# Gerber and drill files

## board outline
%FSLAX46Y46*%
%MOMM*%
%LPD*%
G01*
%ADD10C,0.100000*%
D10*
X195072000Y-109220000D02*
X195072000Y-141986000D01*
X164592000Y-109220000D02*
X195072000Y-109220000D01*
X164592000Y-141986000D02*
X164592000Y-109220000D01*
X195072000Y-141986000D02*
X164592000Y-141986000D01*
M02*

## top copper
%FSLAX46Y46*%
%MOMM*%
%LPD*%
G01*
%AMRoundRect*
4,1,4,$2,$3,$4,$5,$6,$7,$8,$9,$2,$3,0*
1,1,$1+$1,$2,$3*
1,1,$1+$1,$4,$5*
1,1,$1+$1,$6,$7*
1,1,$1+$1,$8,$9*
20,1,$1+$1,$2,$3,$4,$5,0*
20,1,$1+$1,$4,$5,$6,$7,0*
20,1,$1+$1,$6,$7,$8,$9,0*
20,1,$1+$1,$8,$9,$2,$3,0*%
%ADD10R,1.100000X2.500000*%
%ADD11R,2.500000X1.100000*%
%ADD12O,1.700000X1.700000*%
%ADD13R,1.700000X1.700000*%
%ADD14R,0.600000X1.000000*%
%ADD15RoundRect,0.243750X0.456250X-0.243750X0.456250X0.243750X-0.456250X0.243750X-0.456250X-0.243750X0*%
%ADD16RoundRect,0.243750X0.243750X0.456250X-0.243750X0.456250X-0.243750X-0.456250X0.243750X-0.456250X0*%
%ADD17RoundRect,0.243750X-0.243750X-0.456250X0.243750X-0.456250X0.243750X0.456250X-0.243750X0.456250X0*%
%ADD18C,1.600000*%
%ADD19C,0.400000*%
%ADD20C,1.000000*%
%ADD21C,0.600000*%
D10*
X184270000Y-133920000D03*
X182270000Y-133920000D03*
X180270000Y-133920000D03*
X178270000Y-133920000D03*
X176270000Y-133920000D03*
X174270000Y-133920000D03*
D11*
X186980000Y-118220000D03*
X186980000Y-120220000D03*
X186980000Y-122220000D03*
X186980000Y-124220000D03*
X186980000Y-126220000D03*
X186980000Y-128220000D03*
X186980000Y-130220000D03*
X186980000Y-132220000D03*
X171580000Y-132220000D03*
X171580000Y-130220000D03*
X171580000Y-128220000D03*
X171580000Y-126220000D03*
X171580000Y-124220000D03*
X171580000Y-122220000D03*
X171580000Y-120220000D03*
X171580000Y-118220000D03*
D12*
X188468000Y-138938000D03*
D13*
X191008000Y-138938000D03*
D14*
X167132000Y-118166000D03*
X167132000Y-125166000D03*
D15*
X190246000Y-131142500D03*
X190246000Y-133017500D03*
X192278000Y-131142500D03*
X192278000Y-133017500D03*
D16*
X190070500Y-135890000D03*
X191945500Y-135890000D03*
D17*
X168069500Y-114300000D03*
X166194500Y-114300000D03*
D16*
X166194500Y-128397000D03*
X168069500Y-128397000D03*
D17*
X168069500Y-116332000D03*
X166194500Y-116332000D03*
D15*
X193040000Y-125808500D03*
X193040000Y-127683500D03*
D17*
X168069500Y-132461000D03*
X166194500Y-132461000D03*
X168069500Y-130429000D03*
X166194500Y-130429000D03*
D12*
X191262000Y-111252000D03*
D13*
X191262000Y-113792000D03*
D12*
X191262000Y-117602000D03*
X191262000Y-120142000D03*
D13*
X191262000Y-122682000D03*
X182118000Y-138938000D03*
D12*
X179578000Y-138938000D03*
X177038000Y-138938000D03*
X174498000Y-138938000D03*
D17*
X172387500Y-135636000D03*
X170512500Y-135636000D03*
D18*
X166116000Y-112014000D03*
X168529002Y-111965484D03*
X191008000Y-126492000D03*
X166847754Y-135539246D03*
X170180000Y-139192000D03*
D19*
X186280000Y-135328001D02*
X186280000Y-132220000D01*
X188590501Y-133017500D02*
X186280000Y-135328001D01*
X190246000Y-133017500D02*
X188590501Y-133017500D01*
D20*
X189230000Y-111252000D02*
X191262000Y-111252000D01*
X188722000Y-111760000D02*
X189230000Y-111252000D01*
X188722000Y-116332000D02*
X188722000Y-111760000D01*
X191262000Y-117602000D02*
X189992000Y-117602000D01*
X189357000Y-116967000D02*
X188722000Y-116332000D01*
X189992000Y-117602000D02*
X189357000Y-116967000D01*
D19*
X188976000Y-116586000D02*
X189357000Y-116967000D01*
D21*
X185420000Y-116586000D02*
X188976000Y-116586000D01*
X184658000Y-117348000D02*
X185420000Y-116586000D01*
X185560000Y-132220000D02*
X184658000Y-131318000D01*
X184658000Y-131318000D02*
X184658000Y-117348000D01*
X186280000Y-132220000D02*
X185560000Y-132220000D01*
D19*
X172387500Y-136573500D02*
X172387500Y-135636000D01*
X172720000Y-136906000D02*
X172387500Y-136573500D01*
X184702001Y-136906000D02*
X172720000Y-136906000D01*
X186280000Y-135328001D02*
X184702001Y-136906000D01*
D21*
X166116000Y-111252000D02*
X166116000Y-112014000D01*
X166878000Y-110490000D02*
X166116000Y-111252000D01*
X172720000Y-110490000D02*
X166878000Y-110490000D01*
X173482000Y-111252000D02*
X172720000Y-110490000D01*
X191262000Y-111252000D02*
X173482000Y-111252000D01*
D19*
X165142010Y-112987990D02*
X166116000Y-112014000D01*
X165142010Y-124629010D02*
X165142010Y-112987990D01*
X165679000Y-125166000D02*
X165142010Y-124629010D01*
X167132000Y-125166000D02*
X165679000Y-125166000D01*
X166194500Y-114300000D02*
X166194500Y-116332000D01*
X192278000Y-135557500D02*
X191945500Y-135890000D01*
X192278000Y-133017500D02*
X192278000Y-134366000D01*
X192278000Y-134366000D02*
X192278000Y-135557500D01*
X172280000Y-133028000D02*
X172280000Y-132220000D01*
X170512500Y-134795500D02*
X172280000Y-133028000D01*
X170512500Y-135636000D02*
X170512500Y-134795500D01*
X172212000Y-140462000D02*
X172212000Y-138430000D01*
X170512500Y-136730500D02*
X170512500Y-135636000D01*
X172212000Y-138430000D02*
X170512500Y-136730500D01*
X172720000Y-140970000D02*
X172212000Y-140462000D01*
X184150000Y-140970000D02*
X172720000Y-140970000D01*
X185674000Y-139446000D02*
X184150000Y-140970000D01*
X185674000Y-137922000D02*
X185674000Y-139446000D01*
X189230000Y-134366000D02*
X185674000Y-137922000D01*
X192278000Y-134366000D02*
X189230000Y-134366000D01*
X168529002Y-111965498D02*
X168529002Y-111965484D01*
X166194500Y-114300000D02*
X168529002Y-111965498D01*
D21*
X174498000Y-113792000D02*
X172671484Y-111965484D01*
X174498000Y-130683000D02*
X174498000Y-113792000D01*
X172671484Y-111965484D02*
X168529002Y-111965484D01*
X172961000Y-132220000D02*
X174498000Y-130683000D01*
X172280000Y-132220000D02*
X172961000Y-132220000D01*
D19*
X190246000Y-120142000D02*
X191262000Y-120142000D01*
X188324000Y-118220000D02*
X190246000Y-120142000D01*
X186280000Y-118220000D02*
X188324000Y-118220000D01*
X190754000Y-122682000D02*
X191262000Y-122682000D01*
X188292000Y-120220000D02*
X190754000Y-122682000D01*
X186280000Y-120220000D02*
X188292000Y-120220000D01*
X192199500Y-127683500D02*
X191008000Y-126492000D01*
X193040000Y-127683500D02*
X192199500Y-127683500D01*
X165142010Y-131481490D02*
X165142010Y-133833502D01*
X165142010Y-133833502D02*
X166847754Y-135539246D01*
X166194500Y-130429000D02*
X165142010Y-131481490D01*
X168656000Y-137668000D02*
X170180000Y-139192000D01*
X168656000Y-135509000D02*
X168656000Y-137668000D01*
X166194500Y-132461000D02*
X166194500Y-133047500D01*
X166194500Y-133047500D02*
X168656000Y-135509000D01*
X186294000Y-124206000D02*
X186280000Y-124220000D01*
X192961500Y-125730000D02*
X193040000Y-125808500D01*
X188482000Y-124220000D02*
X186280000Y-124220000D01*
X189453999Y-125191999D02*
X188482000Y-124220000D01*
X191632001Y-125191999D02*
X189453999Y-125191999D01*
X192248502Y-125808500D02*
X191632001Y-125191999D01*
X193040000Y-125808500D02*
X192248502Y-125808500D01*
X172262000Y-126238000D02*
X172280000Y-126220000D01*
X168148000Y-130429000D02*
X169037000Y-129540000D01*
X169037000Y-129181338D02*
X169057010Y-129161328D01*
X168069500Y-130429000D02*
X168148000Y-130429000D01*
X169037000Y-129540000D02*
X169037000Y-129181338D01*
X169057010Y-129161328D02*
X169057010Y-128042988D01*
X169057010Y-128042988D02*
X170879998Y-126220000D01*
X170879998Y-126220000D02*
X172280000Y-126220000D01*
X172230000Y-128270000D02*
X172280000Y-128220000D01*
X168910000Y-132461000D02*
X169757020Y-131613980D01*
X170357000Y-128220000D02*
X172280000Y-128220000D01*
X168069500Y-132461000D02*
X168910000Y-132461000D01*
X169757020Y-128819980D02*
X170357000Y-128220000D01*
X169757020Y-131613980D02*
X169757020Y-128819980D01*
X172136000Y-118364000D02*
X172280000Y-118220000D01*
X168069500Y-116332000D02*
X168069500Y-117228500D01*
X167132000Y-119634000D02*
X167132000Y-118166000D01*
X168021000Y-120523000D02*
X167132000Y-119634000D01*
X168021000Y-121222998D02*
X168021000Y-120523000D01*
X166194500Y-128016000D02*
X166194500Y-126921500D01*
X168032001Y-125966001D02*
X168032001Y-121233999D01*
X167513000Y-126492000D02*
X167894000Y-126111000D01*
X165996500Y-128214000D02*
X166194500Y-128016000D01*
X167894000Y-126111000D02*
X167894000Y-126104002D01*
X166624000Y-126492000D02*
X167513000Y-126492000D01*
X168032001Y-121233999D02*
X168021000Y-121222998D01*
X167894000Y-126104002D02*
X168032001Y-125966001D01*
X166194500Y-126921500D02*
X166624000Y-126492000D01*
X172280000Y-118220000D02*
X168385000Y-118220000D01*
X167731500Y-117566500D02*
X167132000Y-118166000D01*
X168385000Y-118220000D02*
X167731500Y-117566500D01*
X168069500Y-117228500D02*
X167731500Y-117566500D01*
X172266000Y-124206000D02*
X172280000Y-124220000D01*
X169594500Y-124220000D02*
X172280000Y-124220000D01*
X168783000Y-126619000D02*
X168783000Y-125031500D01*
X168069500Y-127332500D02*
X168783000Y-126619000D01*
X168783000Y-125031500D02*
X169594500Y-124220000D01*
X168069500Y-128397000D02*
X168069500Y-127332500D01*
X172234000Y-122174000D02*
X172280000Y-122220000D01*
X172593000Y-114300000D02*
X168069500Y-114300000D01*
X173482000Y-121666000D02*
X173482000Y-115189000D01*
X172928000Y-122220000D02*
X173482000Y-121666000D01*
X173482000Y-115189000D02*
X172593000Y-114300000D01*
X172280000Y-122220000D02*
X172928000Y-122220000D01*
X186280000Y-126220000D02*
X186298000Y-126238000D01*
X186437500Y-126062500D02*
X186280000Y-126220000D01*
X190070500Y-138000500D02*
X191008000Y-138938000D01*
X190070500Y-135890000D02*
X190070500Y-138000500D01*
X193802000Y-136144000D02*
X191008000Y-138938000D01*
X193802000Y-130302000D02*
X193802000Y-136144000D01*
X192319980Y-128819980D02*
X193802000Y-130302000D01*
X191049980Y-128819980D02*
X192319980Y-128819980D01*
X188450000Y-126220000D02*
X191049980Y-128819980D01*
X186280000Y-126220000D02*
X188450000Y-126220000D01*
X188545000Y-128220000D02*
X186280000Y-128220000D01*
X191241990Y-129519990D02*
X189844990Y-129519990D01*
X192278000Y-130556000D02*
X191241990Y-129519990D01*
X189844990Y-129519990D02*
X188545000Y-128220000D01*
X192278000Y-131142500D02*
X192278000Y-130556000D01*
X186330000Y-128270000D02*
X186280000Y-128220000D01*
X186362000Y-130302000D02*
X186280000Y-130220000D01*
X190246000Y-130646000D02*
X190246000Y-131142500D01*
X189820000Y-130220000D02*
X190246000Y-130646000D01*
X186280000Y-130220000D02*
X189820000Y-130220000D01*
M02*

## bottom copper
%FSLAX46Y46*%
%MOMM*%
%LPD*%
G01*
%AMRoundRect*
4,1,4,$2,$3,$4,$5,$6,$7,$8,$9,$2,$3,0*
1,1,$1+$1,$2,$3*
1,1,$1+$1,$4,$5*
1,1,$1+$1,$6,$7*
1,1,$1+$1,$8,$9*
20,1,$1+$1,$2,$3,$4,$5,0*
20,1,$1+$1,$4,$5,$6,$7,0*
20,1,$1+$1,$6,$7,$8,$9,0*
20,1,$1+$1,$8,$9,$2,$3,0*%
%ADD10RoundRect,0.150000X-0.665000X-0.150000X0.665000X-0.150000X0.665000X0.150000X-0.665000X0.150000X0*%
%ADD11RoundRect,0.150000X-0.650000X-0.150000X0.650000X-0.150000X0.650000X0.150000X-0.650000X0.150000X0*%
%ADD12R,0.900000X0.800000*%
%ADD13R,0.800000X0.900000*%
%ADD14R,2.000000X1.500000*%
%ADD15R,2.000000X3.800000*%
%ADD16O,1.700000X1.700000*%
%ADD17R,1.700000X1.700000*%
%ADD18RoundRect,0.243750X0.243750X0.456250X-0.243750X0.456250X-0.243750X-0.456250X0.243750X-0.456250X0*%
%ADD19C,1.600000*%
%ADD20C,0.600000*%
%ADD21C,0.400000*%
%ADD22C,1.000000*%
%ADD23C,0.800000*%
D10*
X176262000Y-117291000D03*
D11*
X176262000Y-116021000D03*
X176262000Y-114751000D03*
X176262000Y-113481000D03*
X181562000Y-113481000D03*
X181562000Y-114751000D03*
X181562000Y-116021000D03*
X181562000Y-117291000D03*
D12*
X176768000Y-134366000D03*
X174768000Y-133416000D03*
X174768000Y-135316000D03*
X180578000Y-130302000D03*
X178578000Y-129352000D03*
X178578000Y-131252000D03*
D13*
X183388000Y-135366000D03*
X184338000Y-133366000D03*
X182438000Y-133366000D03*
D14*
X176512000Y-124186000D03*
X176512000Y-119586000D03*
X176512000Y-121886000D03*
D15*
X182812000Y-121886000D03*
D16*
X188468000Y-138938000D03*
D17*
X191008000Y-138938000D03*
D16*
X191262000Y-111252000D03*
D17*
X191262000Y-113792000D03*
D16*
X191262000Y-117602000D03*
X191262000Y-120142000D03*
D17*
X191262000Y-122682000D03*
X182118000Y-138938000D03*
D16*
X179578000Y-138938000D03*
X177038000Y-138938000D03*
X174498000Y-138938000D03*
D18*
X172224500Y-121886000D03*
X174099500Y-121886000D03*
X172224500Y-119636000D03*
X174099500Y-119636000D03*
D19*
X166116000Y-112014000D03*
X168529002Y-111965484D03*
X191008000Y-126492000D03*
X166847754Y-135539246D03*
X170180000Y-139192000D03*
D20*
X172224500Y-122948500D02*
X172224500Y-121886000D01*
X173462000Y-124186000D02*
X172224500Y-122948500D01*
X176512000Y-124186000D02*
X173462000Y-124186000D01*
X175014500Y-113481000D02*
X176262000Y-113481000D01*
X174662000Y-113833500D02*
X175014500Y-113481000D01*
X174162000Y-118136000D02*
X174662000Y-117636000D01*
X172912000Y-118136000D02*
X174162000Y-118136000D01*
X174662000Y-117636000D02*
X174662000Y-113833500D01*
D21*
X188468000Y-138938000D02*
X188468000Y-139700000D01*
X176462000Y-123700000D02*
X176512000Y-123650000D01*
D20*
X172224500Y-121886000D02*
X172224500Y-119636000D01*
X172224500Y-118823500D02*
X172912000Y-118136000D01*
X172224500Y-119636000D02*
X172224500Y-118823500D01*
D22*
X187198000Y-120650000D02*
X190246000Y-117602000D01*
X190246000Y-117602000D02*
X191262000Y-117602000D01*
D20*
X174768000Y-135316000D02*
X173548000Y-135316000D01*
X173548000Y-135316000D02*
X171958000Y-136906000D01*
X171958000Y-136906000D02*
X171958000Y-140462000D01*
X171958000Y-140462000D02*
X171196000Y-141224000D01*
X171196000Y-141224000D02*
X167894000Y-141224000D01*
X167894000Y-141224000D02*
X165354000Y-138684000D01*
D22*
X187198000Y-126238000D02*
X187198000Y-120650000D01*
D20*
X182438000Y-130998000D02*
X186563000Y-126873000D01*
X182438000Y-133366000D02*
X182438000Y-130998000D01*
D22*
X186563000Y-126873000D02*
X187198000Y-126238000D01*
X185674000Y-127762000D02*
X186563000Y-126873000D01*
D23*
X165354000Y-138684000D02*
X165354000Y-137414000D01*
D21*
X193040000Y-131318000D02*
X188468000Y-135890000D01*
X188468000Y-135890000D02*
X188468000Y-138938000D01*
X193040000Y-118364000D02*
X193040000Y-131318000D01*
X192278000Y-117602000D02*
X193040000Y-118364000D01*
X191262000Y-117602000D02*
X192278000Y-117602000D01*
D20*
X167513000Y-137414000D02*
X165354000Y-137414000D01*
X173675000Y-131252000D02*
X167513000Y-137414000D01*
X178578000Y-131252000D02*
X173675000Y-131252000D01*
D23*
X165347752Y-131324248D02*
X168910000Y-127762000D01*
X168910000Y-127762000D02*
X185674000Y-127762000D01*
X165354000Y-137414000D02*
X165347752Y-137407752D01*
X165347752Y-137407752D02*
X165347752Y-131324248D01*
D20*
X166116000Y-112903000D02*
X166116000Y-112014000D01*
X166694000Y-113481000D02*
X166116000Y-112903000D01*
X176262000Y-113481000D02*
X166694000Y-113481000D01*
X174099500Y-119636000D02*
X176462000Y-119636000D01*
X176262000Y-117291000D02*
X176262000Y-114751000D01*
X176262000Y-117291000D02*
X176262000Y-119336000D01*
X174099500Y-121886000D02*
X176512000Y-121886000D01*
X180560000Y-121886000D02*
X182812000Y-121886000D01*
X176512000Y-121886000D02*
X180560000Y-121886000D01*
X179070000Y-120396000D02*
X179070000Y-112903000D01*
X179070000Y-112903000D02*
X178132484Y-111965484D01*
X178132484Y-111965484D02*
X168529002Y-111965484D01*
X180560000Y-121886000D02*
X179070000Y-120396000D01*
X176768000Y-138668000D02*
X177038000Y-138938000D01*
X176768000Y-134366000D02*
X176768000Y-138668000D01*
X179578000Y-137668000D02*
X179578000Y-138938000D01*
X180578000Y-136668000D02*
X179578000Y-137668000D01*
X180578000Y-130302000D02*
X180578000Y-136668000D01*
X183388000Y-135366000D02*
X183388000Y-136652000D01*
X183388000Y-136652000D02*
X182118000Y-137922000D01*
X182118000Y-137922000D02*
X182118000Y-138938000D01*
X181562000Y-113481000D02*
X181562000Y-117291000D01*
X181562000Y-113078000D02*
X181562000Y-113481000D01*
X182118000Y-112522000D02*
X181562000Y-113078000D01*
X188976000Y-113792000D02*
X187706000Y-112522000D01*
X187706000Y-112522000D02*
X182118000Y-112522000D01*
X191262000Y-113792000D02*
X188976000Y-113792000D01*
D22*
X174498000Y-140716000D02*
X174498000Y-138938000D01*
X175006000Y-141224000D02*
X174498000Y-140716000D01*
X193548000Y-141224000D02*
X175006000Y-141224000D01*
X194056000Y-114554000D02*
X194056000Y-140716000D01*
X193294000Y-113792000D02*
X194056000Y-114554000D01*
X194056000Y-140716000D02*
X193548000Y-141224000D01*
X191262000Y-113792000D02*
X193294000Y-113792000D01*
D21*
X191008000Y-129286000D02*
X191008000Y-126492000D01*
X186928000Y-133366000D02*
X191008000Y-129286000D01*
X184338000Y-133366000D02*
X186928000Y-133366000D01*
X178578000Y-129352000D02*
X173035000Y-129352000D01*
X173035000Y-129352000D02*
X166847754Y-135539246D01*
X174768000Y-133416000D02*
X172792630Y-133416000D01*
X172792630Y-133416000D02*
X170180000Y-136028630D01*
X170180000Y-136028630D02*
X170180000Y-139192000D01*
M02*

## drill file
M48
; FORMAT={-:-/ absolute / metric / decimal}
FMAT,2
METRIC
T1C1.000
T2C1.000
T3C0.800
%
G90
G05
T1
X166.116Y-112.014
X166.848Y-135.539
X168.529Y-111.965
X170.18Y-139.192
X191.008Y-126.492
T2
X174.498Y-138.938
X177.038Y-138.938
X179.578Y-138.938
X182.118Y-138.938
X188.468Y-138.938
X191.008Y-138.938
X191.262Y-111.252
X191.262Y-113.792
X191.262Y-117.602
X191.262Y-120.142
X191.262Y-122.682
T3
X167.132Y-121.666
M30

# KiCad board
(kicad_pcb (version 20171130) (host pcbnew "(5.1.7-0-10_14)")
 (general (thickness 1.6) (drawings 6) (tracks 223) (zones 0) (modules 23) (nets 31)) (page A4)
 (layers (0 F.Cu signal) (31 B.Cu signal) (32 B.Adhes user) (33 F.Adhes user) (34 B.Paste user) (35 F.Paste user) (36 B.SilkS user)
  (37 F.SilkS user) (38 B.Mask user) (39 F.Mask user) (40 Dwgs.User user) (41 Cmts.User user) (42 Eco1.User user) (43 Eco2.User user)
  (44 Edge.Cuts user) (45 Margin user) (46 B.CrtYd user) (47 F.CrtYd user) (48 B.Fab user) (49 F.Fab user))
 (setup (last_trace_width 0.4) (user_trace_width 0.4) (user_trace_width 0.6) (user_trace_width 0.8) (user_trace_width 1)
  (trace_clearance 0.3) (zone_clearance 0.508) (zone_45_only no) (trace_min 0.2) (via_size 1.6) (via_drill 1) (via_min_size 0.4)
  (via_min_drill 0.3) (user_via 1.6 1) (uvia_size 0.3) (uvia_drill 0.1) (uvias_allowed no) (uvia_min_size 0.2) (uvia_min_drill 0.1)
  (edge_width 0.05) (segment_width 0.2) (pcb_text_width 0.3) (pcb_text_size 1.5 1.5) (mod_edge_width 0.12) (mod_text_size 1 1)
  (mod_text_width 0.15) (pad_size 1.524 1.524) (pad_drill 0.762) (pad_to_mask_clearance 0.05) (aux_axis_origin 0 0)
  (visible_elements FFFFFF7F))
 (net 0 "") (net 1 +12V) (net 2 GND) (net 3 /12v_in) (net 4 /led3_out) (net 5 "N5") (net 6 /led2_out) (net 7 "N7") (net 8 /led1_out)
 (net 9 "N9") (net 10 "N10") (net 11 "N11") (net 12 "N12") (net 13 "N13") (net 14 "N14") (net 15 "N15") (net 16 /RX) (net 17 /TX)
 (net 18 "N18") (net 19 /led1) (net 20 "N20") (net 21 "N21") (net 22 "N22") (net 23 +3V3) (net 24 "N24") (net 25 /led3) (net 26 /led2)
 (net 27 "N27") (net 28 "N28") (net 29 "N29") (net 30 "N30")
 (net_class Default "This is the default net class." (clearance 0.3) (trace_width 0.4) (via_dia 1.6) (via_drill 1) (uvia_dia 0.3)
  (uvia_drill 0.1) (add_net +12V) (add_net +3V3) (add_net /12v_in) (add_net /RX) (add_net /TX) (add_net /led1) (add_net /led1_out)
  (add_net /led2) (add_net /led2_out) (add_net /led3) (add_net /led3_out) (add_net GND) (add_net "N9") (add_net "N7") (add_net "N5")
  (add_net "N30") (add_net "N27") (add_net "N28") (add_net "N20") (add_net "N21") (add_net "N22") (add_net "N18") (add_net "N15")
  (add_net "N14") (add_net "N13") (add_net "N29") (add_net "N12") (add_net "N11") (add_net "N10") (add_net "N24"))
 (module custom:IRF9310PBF (layer B.Cu) (at 178.912 115.386)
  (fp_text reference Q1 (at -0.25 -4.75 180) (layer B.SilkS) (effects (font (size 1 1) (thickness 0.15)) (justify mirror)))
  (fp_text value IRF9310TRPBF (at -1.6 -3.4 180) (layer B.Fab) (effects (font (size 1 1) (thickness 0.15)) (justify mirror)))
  (pad 3 smd roundrect (at -2.65 1.905) (size 1.63 0.6) (layers B.Cu B.Paste B.Mask) (roundrect_rratio 0.25) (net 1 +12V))
  (pad 3 smd roundrect (at -2.65 0.635) (size 1.6 0.6) (layers B.Cu B.Paste B.Mask) (roundrect_rratio 0.25) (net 1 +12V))
  (pad 3 smd roundrect (at -2.65 -0.635) (size 1.6 0.6) (layers B.Cu B.Paste B.Mask) (roundrect_rratio 0.25) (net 1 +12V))
  (pad 2 smd roundrect (at -2.65 -1.905) (size 1.6 0.6) (layers B.Cu B.Paste B.Mask) (roundrect_rratio 0.25) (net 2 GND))
  (pad 1 smd roundrect (at 2.65 -1.905) (size 1.6 0.6) (layers B.Cu B.Paste B.Mask) (roundrect_rratio 0.25) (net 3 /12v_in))
  (pad 1 smd roundrect (at 2.65 -0.635) (size 1.6 0.6) (layers B.Cu B.Paste B.Mask) (roundrect_rratio 0.25) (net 3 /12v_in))
  (pad 1 smd roundrect (at 2.65 0.635) (size 1.6 0.6) (layers B.Cu B.Paste B.Mask) (roundrect_rratio 0.25) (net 3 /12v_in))
  (pad 1 smd roundrect (at 2.65 1.905) (size 1.6 0.6) (layers B.Cu B.Paste B.Mask) (roundrect_rratio 0.25) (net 3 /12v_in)))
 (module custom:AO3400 (layer B.Cu) (at 175.768 134.366)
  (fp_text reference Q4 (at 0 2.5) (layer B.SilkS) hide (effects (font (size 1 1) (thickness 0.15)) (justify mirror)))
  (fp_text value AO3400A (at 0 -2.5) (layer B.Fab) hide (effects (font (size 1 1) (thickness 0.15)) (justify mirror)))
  (pad 1 smd rect (at 1 0) (size 0.9 0.8) (layers B.Cu B.Paste B.Mask) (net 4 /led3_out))
  (pad 2 smd rect (at -1 -0.95) (size 0.9 0.8) (layers B.Cu B.Paste B.Mask) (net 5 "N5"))
  (pad 3 smd rect (at -1 0.95) (size 0.9 0.8) (layers B.Cu B.Paste B.Mask) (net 2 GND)))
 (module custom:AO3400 (layer B.Cu) (at 179.578 130.302)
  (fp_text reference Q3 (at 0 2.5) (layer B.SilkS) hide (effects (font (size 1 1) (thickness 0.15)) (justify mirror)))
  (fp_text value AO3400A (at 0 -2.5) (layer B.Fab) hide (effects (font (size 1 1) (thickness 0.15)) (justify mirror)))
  (pad 1 smd rect (at 1 0) (size 0.9 0.8) (layers B.Cu B.Paste B.Mask) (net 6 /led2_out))
  (pad 2 smd rect (at -1 -0.95) (size 0.9 0.8) (layers B.Cu B.Paste B.Mask) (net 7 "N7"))
  (pad 3 smd rect (at -1 0.95) (size 0.9 0.8) (layers B.Cu B.Paste B.Mask) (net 2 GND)))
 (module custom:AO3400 (layer B.Cu) (at 183.388 134.366 270)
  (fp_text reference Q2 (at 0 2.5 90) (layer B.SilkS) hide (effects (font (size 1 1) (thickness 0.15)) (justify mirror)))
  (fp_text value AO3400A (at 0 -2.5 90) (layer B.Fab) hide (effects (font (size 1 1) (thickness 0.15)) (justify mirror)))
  (pad 1 smd rect (at 1 0 270) (size 0.9 0.8) (layers B.Cu B.Paste B.Mask) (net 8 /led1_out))
  (pad 2 smd rect (at -1 -0.95 270) (size 0.9 0.8) (layers B.Cu B.Paste B.Mask) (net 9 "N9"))
  (pad 3 smd rect (at -1 0.95 270) (size 0.9 0.8) (layers B.Cu B.Paste B.Mask) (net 2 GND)))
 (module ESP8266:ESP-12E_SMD (layer F.Cu) (at 172.28 118.22)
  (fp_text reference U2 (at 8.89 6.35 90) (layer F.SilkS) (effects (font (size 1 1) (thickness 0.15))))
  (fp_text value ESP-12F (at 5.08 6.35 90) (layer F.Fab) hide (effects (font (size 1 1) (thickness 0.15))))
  (pad 22 smd rect (at 11.99 15 90) (size 2.5 1.1) (drill (offset -0.7 0)) (layers F.Cu F.Paste F.Mask) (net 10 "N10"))
  (pad 21 smd rect (at 9.99 15 90) (size 2.5 1.1) (drill (offset -0.7 0)) (layers F.Cu F.Paste F.Mask) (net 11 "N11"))
  (pad 20 smd rect (at 7.99 15 90) (size 2.5 1.1) (drill (offset -0.7 0)) (layers F.Cu F.Paste F.Mask) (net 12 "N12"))
  (pad 19 smd rect (at 5.99 15 90) (size 2.5 1.1) (drill (offset -0.7 0)) (layers F.Cu F.Paste F.Mask) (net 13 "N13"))
  (pad 18 smd rect (at 3.99 15 90) (size 2.5 1.1) (drill (offset -0.7 0)) (layers F.Cu F.Paste F.Mask) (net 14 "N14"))
  (pad 17 smd rect (at 1.99 15 90) (size 2.5 1.1) (drill (offset -0.7 0)) (layers F.Cu F.Paste F.Mask) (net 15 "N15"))
  (pad 16 smd rect (at 14 0) (size 2.5 1.1) (drill (offset 0.7 0)) (layers F.Cu F.Paste F.Mask) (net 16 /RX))
  (pad 15 smd rect (at 14 2) (size 2.5 1.1) (drill (offset 0.7 0)) (layers F.Cu F.Paste F.Mask) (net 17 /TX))
  (pad 14 smd rect (at 14 4) (size 2.5 1.1) (drill (offset 0.7 0)) (layers F.Cu F.Paste F.Mask) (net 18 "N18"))
  (pad 13 smd rect (at 14 6) (size 2.5 1.1) (drill (offset 0.7 0)) (layers F.Cu F.Paste F.Mask) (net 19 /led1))
  (pad 12 smd rect (at 14 8) (size 2.5 1.1) (drill (offset 0.7 0)) (layers F.Cu F.Paste F.Mask) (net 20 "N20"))
  (pad 11 smd rect (at 14 10) (size 2.5 1.1) (drill (offset 0.7 0)) (layers F.Cu F.Paste F.Mask) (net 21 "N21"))
  (pad 10 smd rect (at 14 12) (size 2.5 1.1) (drill (offset 0.7 0)) (layers F.Cu F.Paste F.Mask) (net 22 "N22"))
  (pad 9 smd rect (at 14 14) (size 2.5 1.1) (drill (offset 0.7 0)) (layers F.Cu F.Paste F.Mask) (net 2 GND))
  (pad 8 smd rect (at 0 14) (size 2.5 1.1) (drill (offset -0.7 0)) (layers F.Cu F.Paste F.Mask) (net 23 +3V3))
  (pad 7 smd rect (at 0 12) (size 2.5 1.1) (drill (offset -0.7 0)) (layers F.Cu F.Paste F.Mask) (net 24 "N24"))
  (pad 6 smd rect (at 0 10) (size 2.5 1.1) (drill (offset -0.7 0)) (layers F.Cu F.Paste F.Mask) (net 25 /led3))
  (pad 5 smd rect (at 0 8) (size 2.5 1.1) (drill (offset -0.7 0)) (layers F.Cu F.Paste F.Mask) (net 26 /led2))
  (pad 4 smd rect (at 0 6) (size 2.5 1.1) (drill (offset -0.7 0)) (layers F.Cu F.Paste F.Mask) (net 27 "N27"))
  (pad 3 smd rect (at 0 4) (size 2.5 1.1) (drill (offset -0.7 0)) (layers F.Cu F.Paste F.Mask) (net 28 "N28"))
  (pad 2 smd rect (at 0 2) (size 2.5 1.1) (drill (offset -0.7 0)) (layers F.Cu F.Paste F.Mask) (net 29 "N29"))
  (pad 1 smd rect (at 0 0) (size 2.5 1.1) (drill (offset -0.7 0)) (layers F.Cu F.Paste F.Mask) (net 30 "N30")))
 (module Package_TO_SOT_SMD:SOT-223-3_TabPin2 (layer B.Cu) (at 179.662 121.886)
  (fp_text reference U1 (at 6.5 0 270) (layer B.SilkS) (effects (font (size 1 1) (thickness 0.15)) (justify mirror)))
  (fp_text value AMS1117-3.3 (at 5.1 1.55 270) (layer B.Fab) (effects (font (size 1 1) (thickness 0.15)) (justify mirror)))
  (pad 1 smd rect (at -3.15 2.3) (size 2 1.5) (layers B.Cu B.Paste B.Mask) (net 2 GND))
  (pad 3 smd rect (at -3.15 -2.3) (size 2 1.5) (layers B.Cu B.Paste B.Mask) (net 1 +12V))
  (pad 2 smd rect (at -3.15 0) (size 2 1.5) (layers B.Cu B.Paste B.Mask) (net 23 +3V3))
  (pad 2 smd rect (at 3.15 0) (size 2 3.8) (layers B.Cu B.Paste B.Mask) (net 23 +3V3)))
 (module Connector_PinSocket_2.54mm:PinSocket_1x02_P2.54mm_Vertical (layer F.Cu) (at 191.008 138.938 270)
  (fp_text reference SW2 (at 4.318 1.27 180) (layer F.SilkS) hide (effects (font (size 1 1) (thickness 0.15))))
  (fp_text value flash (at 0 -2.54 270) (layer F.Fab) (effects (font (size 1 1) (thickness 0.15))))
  (pad 2 thru_hole oval (at 0 2.54 270) (size 1.7 1.7) (drill 1) (layers *.Cu *.Mask) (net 2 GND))
  (pad 1 thru_hole rect (at 0 0 270) (size 1.7 1.7) (drill 1) (layers *.Cu *.Mask) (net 20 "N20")))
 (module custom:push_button (layer F.Cu) (at 167.132 121.666 90)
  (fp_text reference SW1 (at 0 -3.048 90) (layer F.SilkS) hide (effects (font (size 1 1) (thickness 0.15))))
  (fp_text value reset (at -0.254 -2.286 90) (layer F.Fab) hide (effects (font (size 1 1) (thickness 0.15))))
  (pad 2 smd rect (at 3.5 0 90) (size 1 0.6) (layers F.Cu F.Paste F.Mask) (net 30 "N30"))
  (pad "" np_thru_hole circle (at 0 0 90) (size 0.8 0.8) (drill 0.8) (layers *.Cu *.Mask))
  (pad 1 smd rect (at -3.5 0 90) (size 1 0.6) (layers F.Cu F.Paste F.Mask) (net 2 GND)))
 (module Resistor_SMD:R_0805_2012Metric (layer F.Cu) (at 190.246 132.08 90)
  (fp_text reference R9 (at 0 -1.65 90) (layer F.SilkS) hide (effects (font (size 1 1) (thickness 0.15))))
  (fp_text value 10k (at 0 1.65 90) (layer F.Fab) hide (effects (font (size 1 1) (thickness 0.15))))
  (pad 2 smd roundrect (at 0.9375 0 90) (size 0.975 1.4) (layers F.Cu F.Paste F.Mask) (roundrect_rratio 0.25) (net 22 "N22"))
  (pad 1 smd roundrect (at -0.9375 0 90) (size 0.975 1.4) (layers F.Cu F.Paste F.Mask) (roundrect_rratio 0.25) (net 2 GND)))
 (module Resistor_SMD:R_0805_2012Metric (layer F.Cu) (at 192.278 132.08 90)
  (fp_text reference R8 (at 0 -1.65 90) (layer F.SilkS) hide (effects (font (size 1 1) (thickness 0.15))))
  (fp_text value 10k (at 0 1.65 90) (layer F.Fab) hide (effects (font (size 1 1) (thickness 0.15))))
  (pad 2 smd roundrect (at 0.9375 0 90) (size 0.975 1.4) (layers F.Cu F.Paste F.Mask) (roundrect_rratio 0.25) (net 21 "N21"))
  (pad 1 smd roundrect (at -0.9375 0 90) (size 0.975 1.4) (layers F.Cu F.Paste F.Mask) (roundrect_rratio 0.25) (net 23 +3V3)))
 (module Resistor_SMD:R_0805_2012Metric (layer F.Cu) (at 191.008 135.89 180)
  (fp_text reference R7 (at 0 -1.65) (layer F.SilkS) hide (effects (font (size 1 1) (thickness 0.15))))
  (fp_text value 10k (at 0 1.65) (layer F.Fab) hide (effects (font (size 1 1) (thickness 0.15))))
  (pad 2 smd roundrect (at 0.9375 0 180) (size 0.975 1.4) (layers F.Cu F.Paste F.Mask) (roundrect_rratio 0.25) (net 20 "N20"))
  (pad 1 smd roundrect (at -0.9375 0 180) (size 0.975 1.4) (layers F.Cu F.Paste F.Mask) (roundrect_rratio 0.25) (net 23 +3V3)))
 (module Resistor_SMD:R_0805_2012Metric (layer F.Cu) (at 167.132 114.3)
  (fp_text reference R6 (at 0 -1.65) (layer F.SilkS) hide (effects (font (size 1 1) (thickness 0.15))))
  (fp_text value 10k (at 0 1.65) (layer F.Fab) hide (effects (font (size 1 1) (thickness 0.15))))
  (pad 2 smd roundrect (at 0.9375 0) (size 0.975 1.4) (layers F.Cu F.Paste F.Mask) (roundrect_rratio 0.25) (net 28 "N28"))
  (pad 1 smd roundrect (at -0.9375 0) (size 0.975 1.4) (layers F.Cu F.Paste F.Mask) (roundrect_rratio 0.25) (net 23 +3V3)))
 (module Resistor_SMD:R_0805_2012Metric (layer F.Cu) (at 167.132 128.397 180)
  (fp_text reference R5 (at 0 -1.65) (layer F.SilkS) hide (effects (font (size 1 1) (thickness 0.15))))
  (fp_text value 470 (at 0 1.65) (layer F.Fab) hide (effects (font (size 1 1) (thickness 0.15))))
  (pad 2 smd roundrect (at 0.9375 0 180) (size 0.975 1.4) (layers F.Cu F.Paste F.Mask) (roundrect_rratio 0.25) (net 30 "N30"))
  (pad 1 smd roundrect (at -0.9375 0 180) (size 0.975 1.4) (layers F.Cu F.Paste F.Mask) (roundrect_rratio 0.25) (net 27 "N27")))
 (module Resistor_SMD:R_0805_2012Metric (layer F.Cu) (at 167.132 116.332)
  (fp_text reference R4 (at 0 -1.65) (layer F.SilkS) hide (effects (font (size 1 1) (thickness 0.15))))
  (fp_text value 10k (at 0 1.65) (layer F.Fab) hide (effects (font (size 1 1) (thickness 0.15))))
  (pad 2 smd roundrect (at 0.9375 0) (size 0.975 1.4) (layers F.Cu F.Paste F.Mask) (roundrect_rratio 0.25) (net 30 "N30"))
  (pad 1 smd roundrect (at -0.9375 0) (size 0.975 1.4) (layers F.Cu F.Paste F.Mask) (roundrect_rratio 0.25) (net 23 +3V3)))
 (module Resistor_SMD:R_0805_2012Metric (layer F.Cu) (at 193.04 126.746 90)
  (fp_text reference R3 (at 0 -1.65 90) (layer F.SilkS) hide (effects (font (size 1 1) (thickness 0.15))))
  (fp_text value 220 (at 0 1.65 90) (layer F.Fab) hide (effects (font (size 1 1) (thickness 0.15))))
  (pad 2 smd roundrect (at 0.9375 0 90) (size 0.975 1.4) (layers F.Cu F.Paste F.Mask) (roundrect_rratio 0.25) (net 19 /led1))
  (pad 1 smd roundrect (at -0.9375 0 90) (size 0.975 1.4) (layers F.Cu F.Paste F.Mask) (roundrect_rratio 0.25) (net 9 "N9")))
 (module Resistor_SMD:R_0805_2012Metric (layer F.Cu) (at 167.132 132.461)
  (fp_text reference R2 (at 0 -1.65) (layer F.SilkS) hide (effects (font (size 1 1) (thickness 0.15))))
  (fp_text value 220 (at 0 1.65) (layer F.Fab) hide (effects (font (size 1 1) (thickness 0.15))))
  (pad 2 smd roundrect (at 0.9375 0) (size 0.975 1.4) (layers F.Cu F.Paste F.Mask) (roundrect_rratio 0.25) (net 25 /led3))
  (pad 1 smd roundrect (at -0.9375 0) (size 0.975 1.4) (layers F.Cu F.Paste F.Mask) (roundrect_rratio 0.25) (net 5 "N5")))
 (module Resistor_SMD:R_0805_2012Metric (layer F.Cu) (at 167.132 130.429)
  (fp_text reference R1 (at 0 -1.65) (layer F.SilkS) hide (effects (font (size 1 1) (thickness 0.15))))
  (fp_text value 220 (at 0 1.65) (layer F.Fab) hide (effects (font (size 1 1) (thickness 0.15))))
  (pad 2 smd roundrect (at 0.9375 0) (size 0.975 1.4) (layers F.Cu F.Paste F.Mask) (roundrect_rratio 0.25) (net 26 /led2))
  (pad 1 smd roundrect (at -0.9375 0) (size 0.975 1.4) (layers F.Cu F.Paste F.Mask) (roundrect_rratio 0.25) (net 7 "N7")))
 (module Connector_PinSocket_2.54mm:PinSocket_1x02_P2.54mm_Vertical (layer F.Cu) (at 191.262 113.792 180)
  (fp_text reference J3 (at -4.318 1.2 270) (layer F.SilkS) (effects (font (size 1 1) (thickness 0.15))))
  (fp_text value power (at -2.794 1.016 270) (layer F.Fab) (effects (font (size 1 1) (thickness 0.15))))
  (pad 2 thru_hole oval (at 0 2.54 180) (size 1.7 1.7) (drill 1) (layers *.Cu *.Mask) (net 2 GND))
  (pad 1 thru_hole rect (at 0 0 180) (size 1.7 1.7) (drill 1) (layers *.Cu *.Mask) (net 3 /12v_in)))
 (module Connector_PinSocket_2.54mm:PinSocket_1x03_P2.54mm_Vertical (layer F.Cu) (at 191.262 122.682 180)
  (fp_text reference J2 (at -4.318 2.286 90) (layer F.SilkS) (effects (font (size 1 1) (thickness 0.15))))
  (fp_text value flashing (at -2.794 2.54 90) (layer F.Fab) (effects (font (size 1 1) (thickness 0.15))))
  (pad 3 thru_hole oval (at 0 5.08 180) (size 1.7 1.7) (drill 1) (layers *.Cu *.Mask) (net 2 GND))
  (pad 2 thru_hole oval (at 0 2.54 180) (size 1.7 1.7) (drill 1) (layers *.Cu *.Mask) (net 16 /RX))
  (pad 1 thru_hole rect (at 0 0 180) (size 1.7 1.7) (drill 1) (layers *.Cu *.Mask) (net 17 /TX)))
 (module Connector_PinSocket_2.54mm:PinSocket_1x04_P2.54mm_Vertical (layer F.Cu) (at 182.118 138.938 270)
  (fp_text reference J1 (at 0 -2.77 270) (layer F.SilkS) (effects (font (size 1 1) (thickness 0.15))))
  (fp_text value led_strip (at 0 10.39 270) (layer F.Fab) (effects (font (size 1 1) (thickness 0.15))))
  (pad 1 thru_hole rect (at 0 0 270) (size 1.7 1.7) (drill 1) (layers *.Cu *.Mask) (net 8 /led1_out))
  (pad 2 thru_hole oval (at 0 2.54 270) (size 1.7 1.7) (drill 1) (layers *.Cu *.Mask) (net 6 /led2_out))
  (pad 3 thru_hole oval (at 0 5.08 270) (size 1.7 1.7) (drill 1) (layers *.Cu *.Mask) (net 4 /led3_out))
  (pad 4 thru_hole oval (at 0 7.62 270) (size 1.7 1.7) (drill 1) (layers *.Cu *.Mask) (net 3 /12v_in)))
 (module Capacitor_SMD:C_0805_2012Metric (layer F.Cu) (at 171.45 135.636)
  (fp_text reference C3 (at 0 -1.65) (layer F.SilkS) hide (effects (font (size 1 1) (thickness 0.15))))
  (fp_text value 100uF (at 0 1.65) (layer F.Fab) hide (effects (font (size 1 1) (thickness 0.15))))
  (pad 2 smd roundrect (at 0.9375 0) (size 0.975 1.4) (layers F.Cu F.Paste F.Mask) (roundrect_rratio 0.25) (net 2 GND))
  (pad 1 smd roundrect (at -0.9375 0) (size 0.975 1.4) (layers F.Cu F.Paste F.Mask) (roundrect_rratio 0.25) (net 23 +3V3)))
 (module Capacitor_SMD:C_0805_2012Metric (layer B.Cu) (at 173.162 121.886 180)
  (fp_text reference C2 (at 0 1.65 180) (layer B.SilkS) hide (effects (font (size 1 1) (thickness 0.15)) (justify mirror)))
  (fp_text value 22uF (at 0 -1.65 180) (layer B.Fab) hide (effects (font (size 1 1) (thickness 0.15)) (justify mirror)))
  (pad 2 smd roundrect (at 0.9375 0 180) (size 0.975 1.4) (layers B.Cu B.Paste B.Mask) (roundrect_rratio 0.25) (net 2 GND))
  (pad 1 smd roundrect (at -0.9375 0 180) (size 0.975 1.4) (layers B.Cu B.Paste B.Mask) (roundrect_rratio 0.25) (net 23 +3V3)))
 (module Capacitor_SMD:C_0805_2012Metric (layer B.Cu) (at 173.162 119.636 180)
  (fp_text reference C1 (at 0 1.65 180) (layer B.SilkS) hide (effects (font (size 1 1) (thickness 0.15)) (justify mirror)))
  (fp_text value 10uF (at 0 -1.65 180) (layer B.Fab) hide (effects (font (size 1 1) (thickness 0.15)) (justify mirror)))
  (pad 2 smd roundrect (at 0.9375 0 180) (size 0.975 1.4) (layers B.Cu B.Paste B.Mask) (roundrect_rratio 0.25) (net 2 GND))
  (pad 1 smd roundrect (at -0.9375 0 180) (size 0.975 1.4) (layers B.Cu B.Paste B.Mask) (roundrect_rratio 0.25) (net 1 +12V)))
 (gr_line (start 195.072 109.22) (end 195.072 141.986) (layer Edge.Cuts) (width 0.1))
 (gr_line (start 164.592 109.22) (end 195.072 109.22) (layer Edge.Cuts) (width 0.1))
 (gr_line (start 164.592 141.986) (end 164.592 109.22) (layer Edge.Cuts) (width 0.1))
 (gr_line (start 195.072 141.986) (end 164.592 141.986) (layer Edge.Cuts) (width 0.1))
 (segment (start 172.2245 122.9485) (end 172.2245 121.886) (width 0.6) (layer B.Cu) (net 2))
 (segment (start 173.462 124.186) (end 172.2245 122.9485) (width 0.6) (layer B.Cu) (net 2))
 (segment (start 176.512 124.186) (end 173.462 124.186) (width 0.6) (layer B.Cu) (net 2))
 (segment (start 175.0145 113.481) (end 176.262 113.481) (width 0.6) (layer B.Cu) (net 2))
 (segment (start 174.662 113.8335) (end 175.0145 113.481) (width 0.6) (layer B.Cu) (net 2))
 (segment (start 174.162 118.136) (end 174.662 117.636) (width 0.6) (layer B.Cu) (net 2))
 (segment (start 172.912 118.136) (end 174.162 118.136) (width 0.6) (layer B.Cu) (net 2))
 (segment (start 174.662 117.636) (end 174.662 113.8335) (width 0.6) (layer B.Cu) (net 2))
 (segment (start 188.468 138.938) (end 188.468 139.7) (width 0.4) (layer B.Cu) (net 2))
 (segment (start 186.28 135.328001) (end 186.28 132.22) (width 0.4) (layer F.Cu) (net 2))
 (segment (start 188.590501 133.0175) (end 186.28 135.328001) (width 0.4) (layer F.Cu) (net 2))
 (segment (start 190.246 133.0175) (end 188.590501 133.0175) (width 0.4) (layer F.Cu) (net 2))
 (segment (start 189.23 111.252) (end 191.262 111.252) (width 1) (layer F.Cu) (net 2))
 (segment (start 188.722 111.76) (end 189.23 111.252) (width 1) (layer F.Cu) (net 2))
 (segment (start 188.722 116.332) (end 188.722 111.76) (width 1) (layer F.Cu) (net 2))
 (segment (start 191.262 117.602) (end 189.992 117.602) (width 1) (layer F.Cu) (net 2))
 (segment (start 189.357 116.967) (end 188.722 116.332) (width 1) (layer F.Cu) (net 2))
 (segment (start 189.992 117.602) (end 189.357 116.967) (width 1) (layer F.Cu) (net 2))
 (segment (start 176.462 123.7) (end 176.512 123.65) (width 0.4) (layer B.Cu) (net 2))
 (segment (start 172.2245 121.886) (end 172.2245 119.636) (width 0.6) (layer B.Cu) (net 2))
 (segment (start 172.2245 118.8235) (end 172.912 118.136) (width 0.6) (layer B.Cu) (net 2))
 (segment (start 172.2245 119.636) (end 172.2245 118.8235) (width 0.6) (layer B.Cu) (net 2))
 (segment (start 188.976 116.586) (end 189.357 116.967) (width 0.4) (layer F.Cu) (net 2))
 (segment (start 185.42 116.586) (end 188.976 116.586) (width 0.6) (layer F.Cu) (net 2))
 (segment (start 184.658 117.348) (end 185.42 116.586) (width 0.6) (layer F.Cu) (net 2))
 (segment (start 185.56 132.22) (end 184.658 131.318) (width 0.6) (layer F.Cu) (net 2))
 (segment (start 184.658 131.318) (end 184.658 117.348) (width 0.6) (layer F.Cu) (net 2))
 (segment (start 186.28 132.22) (end 185.56 132.22) (width 0.6) (layer F.Cu) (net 2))
 (segment (start 172.3875 136.5735) (end 172.3875 135.636) (width 0.4) (layer F.Cu) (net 2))
 (segment (start 172.72 136.906) (end 172.3875 136.5735) (width 0.4) (layer F.Cu) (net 2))
 (segment (start 184.702001 136.906) (end 172.72 136.906) (width 0.4) (layer F.Cu) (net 2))
 (segment (start 186.28 135.328001) (end 184.702001 136.906) (width 0.4) (layer F.Cu) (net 2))
 (segment (start 187.198 120.65) (end 190.246 117.602) (width 1) (layer B.Cu) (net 2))
 (segment (start 190.246 117.602) (end 191.262 117.602) (width 1) (layer B.Cu) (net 2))
 (segment (start 174.768 135.316) (end 173.548 135.316) (width 0.6) (layer B.Cu) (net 2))
 (segment (start 173.548 135.316) (end 171.958 136.906) (width 0.6) (layer B.Cu) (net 2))
 (segment (start 171.958 136.906) (end 171.958 140.462) (width 0.6) (layer B.Cu) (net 2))
 (segment (start 171.958 140.462) (end 171.196 141.224) (width 0.6) (layer B.Cu) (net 2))
 (segment (start 171.196 141.224) (end 167.894 141.224) (width 0.6) (layer B.Cu) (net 2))
 (segment (start 167.894 141.224) (end 165.354 138.684) (width 0.6) (layer B.Cu) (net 2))
 (segment (start 187.198 126.238) (end 187.198 120.65) (width 1) (layer B.Cu) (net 2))
 (segment (start 182.438 130.998) (end 186.563 126.873) (width 0.6) (layer B.Cu) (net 2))
 (segment (start 182.438 133.366) (end 182.438 130.998) (width 0.6) (layer B.Cu) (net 2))
 (segment (start 186.563 126.873) (end 187.198 126.238) (width 1) (layer B.Cu) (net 2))
 (segment (start 185.674 127.762) (end 186.563 126.873) (width 1) (layer B.Cu) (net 2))
 (segment (start 165.354 138.684) (end 165.354 137.414) (width 0.8) (layer B.Cu) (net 2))
 (segment (start 193.04 131.318) (end 188.468 135.89) (width 0.4) (layer B.Cu) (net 2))
 (segment (start 188.468 135.89) (end 188.468 138.938) (width 0.4) (layer B.Cu) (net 2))
 (segment (start 193.04 118.364) (end 193.04 131.318) (width 0.4) (layer B.Cu) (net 2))
 (segment (start 192.278 117.602) (end 193.04 118.364) (width 0.4) (layer B.Cu) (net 2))
 (segment (start 191.262 117.602) (end 192.278 117.602) (width 0.4) (layer B.Cu) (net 2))
 (segment (start 167.513 137.414) (end 165.354 137.414) (width 0.6) (layer B.Cu) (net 2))
 (segment (start 173.675 131.252) (end 167.513 137.414) (width 0.6) (layer B.Cu) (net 2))
 (segment (start 178.578 131.252) (end 173.675 131.252) (width 0.6) (layer B.Cu) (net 2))
 (segment (start 165.347752 131.324248) (end 168.91 127.762) (width 0.8) (layer B.Cu) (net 2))
 (segment (start 168.91 127.762) (end 185.674 127.762) (width 0.8) (layer B.Cu) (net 2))
 (segment (start 165.354 137.414) (end 165.347752 137.407752) (width 0.8) (layer B.Cu) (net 2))
 (segment (start 165.347752 137.407752) (end 165.347752 131.324248) (width 0.8) (layer B.Cu) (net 2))
 (via (at 166.116 112.014) (size 1.6) (drill 1) (layers F.Cu B.Cu) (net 2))
 (segment (start 166.116 112.903) (end 166.116 112.014) (width 0.6) (layer B.Cu) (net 2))
 (segment (start 166.694 113.481) (end 166.116 112.903) (width 0.6) (layer B.Cu) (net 2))
 (segment (start 176.262 113.481) (end 166.694 113.481) (width 0.6) (layer B.Cu) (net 2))
 (segment (start 166.116 111.252) (end 166.116 112.014) (width 0.6) (layer F.Cu) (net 2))
 (segment (start 166.878 110.49) (end 166.116 111.252) (width 0.6) (layer F.Cu) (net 2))
 (segment (start 172.72 110.49) (end 166.878 110.49) (width 0.6) (layer F.Cu) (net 2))
 (segment (start 173.482 111.252) (end 172.72 110.49) (width 0.6) (layer F.Cu) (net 2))
 (segment (start 191.262 111.252) (end 173.482 111.252) (width 0.6) (layer F.Cu) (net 2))
 (segment (start 165.14201 112.98799) (end 166.116 112.014) (width 0.4) (layer F.Cu) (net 2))
 (segment (start 165.14201 124.62901) (end 165.14201 112.98799) (width 0.4) (layer F.Cu) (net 2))
 (segment (start 165.679 125.166) (end 165.14201 124.62901) (width 0.4) (layer F.Cu) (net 2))
 (segment (start 167.132 125.166) (end 165.679 125.166) (width 0.4) (layer F.Cu) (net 2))
 (segment (start 174.0995 119.636) (end 176.462 119.636) (width 0.6) (layer B.Cu) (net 1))
 (segment (start 176.262 117.291) (end 176.262 114.751) (width 0.6) (layer B.Cu) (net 1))
 (segment (start 176.262 117.291) (end 176.262 119.336) (width 0.6) (layer B.Cu) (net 1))
 (segment (start 174.0995 121.886) (end 176.512 121.886) (width 0.6) (layer B.Cu) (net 23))
 (segment (start 166.1945 114.3) (end 166.1945 116.332) (width 0.4) (layer F.Cu) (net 23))
 (segment (start 192.278 135.5575) (end 191.9455 135.89) (width 0.4) (layer F.Cu) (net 23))
 (segment (start 192.278 133.0175) (end 192.278 134.366) (width 0.4) (layer F.Cu) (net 23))
 (segment (start 192.278 134.366) (end 192.278 135.5575) (width 0.4) (layer F.Cu) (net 23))
 (segment (start 180.56 121.886) (end 182.812 121.886) (width 0.6) (layer B.Cu) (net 23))
 (segment (start 176.512 121.886) (end 180.56 121.886) (width 0.6) (layer B.Cu) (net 23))
 (segment (start 172.28 133.028) (end 172.28 132.22) (width 0.4) (layer F.Cu) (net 23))
 (segment (start 170.5125 134.7955) (end 172.28 133.028) (width 0.4) (layer F.Cu) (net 23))
 (segment (start 170.5125 135.636) (end 170.5125 134.7955) (width 0.4) (layer F.Cu) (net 23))
 (segment (start 172.212 140.462) (end 172.212 138.43) (width 0.4) (layer F.Cu) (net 23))
 (segment (start 170.5125 136.7305) (end 170.5125 135.636) (width 0.4) (layer F.Cu) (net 23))
 (segment (start 172.212 138.43) (end 170.5125 136.7305) (width 0.4) (layer F.Cu) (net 23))
 (segment (start 172.72 140.97) (end 172.212 140.462) (width 0.4) (layer F.Cu) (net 23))
 (segment (start 184.15 140.97) (end 172.72 140.97) (width 0.4) (layer F.Cu) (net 23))
 (segment (start 185.674 139.446) (end 184.15 140.97) (width 0.4) (layer F.Cu) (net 23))
 (segment (start 185.674 137.922) (end 185.674 139.446) (width 0.4) (layer F.Cu) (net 23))
 (segment (start 189.23 134.366) (end 185.674 137.922) (width 0.4) (layer F.Cu) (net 23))
 (segment (start 192.278 134.366) (end 189.23 134.366) (width 0.4) (layer F.Cu) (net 23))
 (via (at 168.529002 111.965484) (size 1.6) (drill 1) (layers F.Cu B.Cu) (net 23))
 (segment (start 179.07 120.396) (end 179.07 112.903) (width 0.6) (layer B.Cu) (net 23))
 (segment (start 179.07 112.903) (end 178.132484 111.965484) (width 0.6) (layer B.Cu) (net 23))
 (segment (start 168.529002 111.965498) (end 168.529002 111.965484) (width 0.4) (layer F.Cu) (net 23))
 (segment (start 178.132484 111.965484) (end 168.529002 111.965484) (width 0.6) (layer B.Cu) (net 23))
 (segment (start 166.1945 114.3) (end 168.529002 111.965498) (width 0.4) (layer F.Cu) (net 23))
 (segment (start 180.56 121.886) (end 179.07 120.396) (width 0.6) (layer B.Cu) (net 23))
 (segment (start 174.498 113.792) (end 172.671484 111.965484) (width 0.6) (layer F.Cu) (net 23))
 (segment (start 174.498 130.683) (end 174.498 113.792) (width 0.6) (layer F.Cu) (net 23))
 (segment (start 172.671484 111.965484) (end 168.529002 111.965484) (width 0.6) (layer F.Cu) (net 23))
 (segment (start 172.961 132.22) (end 174.498 130.683) (width 0.6) (layer F.Cu) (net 23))
 (segment (start 172.28 132.22) (end 172.961 132.22) (width 0.6) (layer F.Cu) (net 23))
 (segment (start 176.768 138.668) (end 177.038 138.938) (width 0.6) (layer B.Cu) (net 4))
 (segment (start 176.768 134.366) (end 176.768 138.668) (width 0.6) (layer B.Cu) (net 4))
 (segment (start 179.578 137.668) (end 179.578 138.938) (width 0.6) (layer B.Cu) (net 6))
 (segment (start 180.578 136.668) (end 179.578 137.668) (width 0.6) (layer B.Cu) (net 6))
 (segment (start 180.578 130.302) (end 180.578 136.668) (width 0.6) (layer B.Cu) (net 6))
 (segment (start 183.388 135.366) (end 183.388 136.652) (width 0.6) (layer B.Cu) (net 8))
 (segment (start 183.388 136.652) (end 182.118 137.922) (width 0.6) (layer B.Cu) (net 8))
 (segment (start 182.118 137.922) (end 182.118 138.938) (width 0.6) (layer B.Cu) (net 8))
 (segment (start 190.246 120.142) (end 191.262 120.142) (width 0.4) (layer F.Cu) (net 16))
 (segment (start 188.324 118.22) (end 190.246 120.142) (width 0.4) (layer F.Cu) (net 16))
 (segment (start 186.28 118.22) (end 188.324 118.22) (width 0.4) (layer F.Cu) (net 16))
 (segment (start 190.754 122.682) (end 191.262 122.682) (width 0.4) (layer F.Cu) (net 17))
 (segment (start 188.292 120.22) (end 190.754 122.682) (width 0.4) (layer F.Cu) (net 17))
 (segment (start 186.28 120.22) (end 188.292 120.22) (width 0.4) (layer F.Cu) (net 17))
 (segment (start 181.562 113.481) (end 181.562 117.291) (width 0.6) (layer B.Cu) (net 3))
 (segment (start 181.562 113.078) (end 181.562 113.481) (width 0.6) (layer B.Cu) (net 3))
 (segment (start 182.118 112.522) (end 181.562 113.078) (width 0.6) (layer B.Cu) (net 3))
 (segment (start 188.976 113.792) (end 187.706 112.522) (width 0.6) (layer B.Cu) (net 3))
 (segment (start 187.706 112.522) (end 182.118 112.522) (width 0.6) (layer B.Cu) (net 3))
 (segment (start 191.262 113.792) (end 188.976 113.792) (width 0.6) (layer B.Cu) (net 3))
 (segment (start 174.498 140.716) (end 174.498 138.938) (width 1) (layer B.Cu) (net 3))
 (segment (start 175.006 141.224) (end 174.498 140.716) (width 1) (layer B.Cu) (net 3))
 (segment (start 193.548 141.224) (end 175.006 141.224) (width 1) (layer B.Cu) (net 3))
 (segment (start 194.056 114.554) (end 194.056 140.716) (width 1) (layer B.Cu) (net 3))
 (segment (start 193.294 113.792) (end 194.056 114.554) (width 1) (layer B.Cu) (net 3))
 (segment (start 194.056 140.716) (end 193.548 141.224) (width 1) (layer B.Cu) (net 3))
 (segment (start 191.262 113.792) (end 193.294 113.792) (width 1) (layer B.Cu) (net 3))
 (via (at 191.008 126.492) (size 1.6) (drill 1) (layers F.Cu B.Cu) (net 9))
 (segment (start 192.1995 127.6835) (end 191.008 126.492) (width 0.4) (layer F.Cu) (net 9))
 (segment (start 193.04 127.6835) (end 192.1995 127.6835) (width 0.4) (layer F.Cu) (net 9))
 (segment (start 191.008 129.286) (end 191.008 126.492) (width 0.4) (layer B.Cu) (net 9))
 (segment (start 186.928 133.366) (end 191.008 129.286) (width 0.4) (layer B.Cu) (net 9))
 (segment (start 184.338 133.366) (end 186.928 133.366) (width 0.4) (layer B.Cu) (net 9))
 (via (at 166.847754 135.539246) (size 1.6) (drill 1) (layers F.Cu B.Cu) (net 7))
 (segment (start 165.14201 131.48149) (end 165.14201 133.833502) (width 0.4) (layer F.Cu) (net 7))
 (segment (start 165.14201 133.833502) (end 166.847754 135.539246) (width 0.4) (layer F.Cu) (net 7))
 (segment (start 178.578 129.352) (end 173.035 129.352) (width 0.4) (layer B.Cu) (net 7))
 (segment (start 173.035 129.352) (end 166.847754 135.539246) (width 0.4) (layer B.Cu) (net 7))
 (segment (start 166.1945 130.429) (end 165.14201 131.48149) (width 0.4) (layer F.Cu) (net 7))
 (via (at 170.18 139.192) (size 1.6) (drill 1) (layers F.Cu B.Cu) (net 5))
 (segment (start 174.768 133.416) (end 172.79263 133.416) (width 0.4) (layer B.Cu) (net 5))
 (segment (start 172.79263 133.416) (end 170.18 136.02863) (width 0.4) (layer B.Cu) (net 5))
 (segment (start 170.18 136.02863) (end 170.18 139.192) (width 0.4) (layer B.Cu) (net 5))
 (segment (start 168.656 137.668) (end 170.18 139.192) (width 0.4) (layer F.Cu) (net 5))
 (segment (start 168.656 135.509) (end 168.656 137.668) (width 0.4) (layer F.Cu) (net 5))
 (segment (start 166.1945 132.461) (end 166.1945 133.0475) (width 0.4) (layer F.Cu) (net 5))
 (segment (start 166.1945 133.0475) (end 168.656 135.509) (width 0.4) (layer F.Cu) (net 5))
 (segment (start 186.294 124.206) (end 186.28 124.22) (width 0.4) (layer F.Cu) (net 19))
 (segment (start 192.9615 125.73) (end 193.04 125.8085) (width 0.4) (layer F.Cu) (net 19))
 (segment (start 188.482 124.22) (end 186.28 124.22) (width 0.4) (layer F.Cu) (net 19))
 (segment (start 189.453999 125.191999) (end 188.482 124.22) (width 0.4) (layer F.Cu) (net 19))
 (segment (start 191.632001 125.191999) (end 189.453999 125.191999) (width 0.4) (layer F.Cu) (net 19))
 (segment (start 192.248502 125.8085) (end 191.632001 125.191999) (width 0.4) (layer F.Cu) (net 19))
 (segment (start 193.04 125.8085) (end 192.248502 125.8085) (width 0.4) (layer F.Cu) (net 19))
 (segment (start 172.262 126.238) (end 172.28 126.22) (width 0.4) (layer F.Cu) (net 26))
 (segment (start 168.148 130.429) (end 169.037 129.54) (width 0.4) (layer F.Cu) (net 26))
 (segment (start 169.037 129.181338) (end 169.05701 129.161328) (width 0.4) (layer F.Cu) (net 26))
 (segment (start 168.0695 130.429) (end 168.148 130.429) (width 0.4) (layer F.Cu) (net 26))
 (segment (start 169.037 129.54) (end 169.037 129.181338) (width 0.4) (layer F.Cu) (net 26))
 (segment (start 169.05701 129.161328) (end 169.05701 128.042988) (width 0.4) (layer F.Cu) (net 26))
 (segment (start 169.05701 128.042988) (end 170.879998 126.22) (width 0.4) (layer F.Cu) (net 26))
 (segment (start 170.879998 126.22) (end 172.28 126.22) (width 0.4) (layer F.Cu) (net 26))
 (segment (start 172.23 128.27) (end 172.28 128.22) (width 0.4) (layer F.Cu) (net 25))
 (segment (start 168.91 132.461) (end 169.75702 131.61398) (width 0.4) (layer F.Cu) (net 25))
 (segment (start 170.357 128.22) (end 172.28 128.22) (width 0.4) (layer F.Cu) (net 25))
 (segment (start 168.0695 132.461) (end 168.91 132.461) (width 0.4) (layer F.Cu) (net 25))
 (segment (start 169.75702 128.81998) (end 170.357 128.22) (width 0.4) (layer F.Cu) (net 25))
 (segment (start 169.75702 131.61398) (end 169.75702 128.81998) (width 0.4) (layer F.Cu) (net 25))
 (segment (start 172.136 118.364) (end 172.28 118.22) (width 0.4) (layer F.Cu) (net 30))
 (segment (start 168.0695 116.332) (end 168.0695 117.2285) (width 0.4) (layer F.Cu) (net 30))
 (segment (start 167.132 119.634) (end 167.132 118.166) (width 0.4) (layer F.Cu) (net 30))
 (segment (start 168.021 120.523) (end 167.132 119.634) (width 0.4) (layer F.Cu) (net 30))
 (segment (start 168.021 121.222998) (end 168.021 120.523) (width 0.4) (layer F.Cu) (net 30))
 (segment (start 166.1945 128.016) (end 166.1945 126.9215) (width 0.4) (layer F.Cu) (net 30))
 (segment (start 168.032001 125.966001) (end 168.032001 121.233999) (width 0.4) (layer F.Cu) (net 30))
 (segment (start 167.513 126.492) (end 167.894 126.111) (width 0.4) (layer F.Cu) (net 30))
 (segment (start 165.9965 128.214) (end 166.1945 128.016) (width 0.4) (layer F.Cu) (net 30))
 (segment (start 167.894 126.111) (end 167.894 126.104002) (width 0.4) (layer F.Cu) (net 30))
 (segment (start 166.624 126.492) (end 167.513 126.492) (width 0.4) (layer F.Cu) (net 30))
 (segment (start 168.032001 121.233999) (end 168.021 121.222998) (width 0.4) (layer F.Cu) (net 30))
 (segment (start 167.894 126.104002) (end 168.032001 125.966001) (width 0.4) (layer F.Cu) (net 30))
 (segment (start 166.1945 126.9215) (end 166.624 126.492) (width 0.4) (layer F.Cu) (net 30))
 (segment (start 172.28 118.22) (end 168.385 118.22) (width 0.4) (layer F.Cu) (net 30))
 (segment (start 167.7315 117.5665) (end 167.132 118.166) (width 0.4) (layer F.Cu) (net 30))
 (segment (start 168.385 118.22) (end 167.7315 117.5665) (width 0.4) (layer F.Cu) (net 30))
 (segment (start 168.0695 117.2285) (end 167.7315 117.5665) (width 0.4) (layer F.Cu) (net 30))
 (segment (start 172.266 124.206) (end 172.28 124.22) (width 0.4) (layer F.Cu) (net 27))
 (segment (start 169.5945 124.22) (end 172.28 124.22) (width 0.4) (layer F.Cu) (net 27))
 (segment (start 168.783 126.619) (end 168.783 125.0315) (width 0.4) (layer F.Cu) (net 27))
 (segment (start 168.0695 127.3325) (end 168.783 126.619) (width 0.4) (layer F.Cu) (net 27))
 (segment (start 168.783 125.0315) (end 169.5945 124.22) (width 0.4) (layer F.Cu) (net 27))
 (segment (start 168.0695 128.397) (end 168.0695 127.3325) (width 0.4) (layer F.Cu) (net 27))
 (segment (start 172.234 122.174) (end 172.28 122.22) (width 0.4) (layer F.Cu) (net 28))
 (segment (start 172.593 114.3) (end 168.0695 114.3) (width 0.4) (layer F.Cu) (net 28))
 (segment (start 173.482 121.666) (end 173.482 115.189) (width 0.4) (layer F.Cu) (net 28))
 (segment (start 172.928 122.22) (end 173.482 121.666) (width 0.4) (layer F.Cu) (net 28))
 (segment (start 173.482 115.189) (end 172.593 114.3) (width 0.4) (layer F.Cu) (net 28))
 (segment (start 172.28 122.22) (end 172.928 122.22) (width 0.4) (layer F.Cu) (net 28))
 (segment (start 186.28 126.22) (end 186.298 126.238) (width 0.4) (layer F.Cu) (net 20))
 (segment (start 186.4375 126.0625) (end 186.28 126.22) (width 0.4) (layer F.Cu) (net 20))
 (segment (start 190.0705 138.0005) (end 191.008 138.938) (width 0.4) (layer F.Cu) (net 20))
 (segment (start 190.0705 135.89) (end 190.0705 138.0005) (width 0.4) (layer F.Cu) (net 20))
 (segment (start 193.802 136.144) (end 191.008 138.938) (width 0.4) (layer F.Cu) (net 20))
 (segment (start 193.802 130.302) (end 193.802 136.144) (width 0.4) (layer F.Cu) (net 20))
 (segment (start 192.31998 128.81998) (end 193.802 130.302) (width 0.4) (layer F.Cu) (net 20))
 (segment (start 191.04998 128.81998) (end 192.31998 128.81998) (width 0.4) (layer F.Cu) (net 20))
 (segment (start 188.45 126.22) (end 191.04998 128.81998) (width 0.4) (layer F.Cu) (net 20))
 (segment (start 186.28 126.22) (end 188.45 126.22) (width 0.4) (layer F.Cu) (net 20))
 (segment (start 188.545 128.22) (end 186.28 128.22) (width 0.4) (layer F.Cu) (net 21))
 (segment (start 191.24199 129.51999) (end 189.84499 129.51999) (width 0.4) (layer F.Cu) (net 21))
 (segment (start 192.278 130.556) (end 191.24199 129.51999) (width 0.4) (layer F.Cu) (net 21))
 (segment (start 189.84499 129.51999) (end 188.545 128.22) (width 0.4) (layer F.Cu) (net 21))
 (segment (start 192.278 131.1425) (end 192.278 130.556) (width 0.4) (layer F.Cu) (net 21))
 (segment (start 186.33 128.27) (end 186.28 128.22) (width 0.4) (layer F.Cu) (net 21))
 (segment (start 186.362 130.302) (end 186.28 130.22) (width 0.4) (layer F.Cu) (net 22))
 (segment (start 190.246 130.646) (end 190.246 131.1425) (width 0.4) (layer F.Cu) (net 22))
 (segment (start 189.82 130.22) (end 190.246 130.646) (width 0.4) (layer F.Cu) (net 22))
 (segment (start 186.28 130.22) (end 189.82 130.22) (width 0.4) (layer F.Cu) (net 22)))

